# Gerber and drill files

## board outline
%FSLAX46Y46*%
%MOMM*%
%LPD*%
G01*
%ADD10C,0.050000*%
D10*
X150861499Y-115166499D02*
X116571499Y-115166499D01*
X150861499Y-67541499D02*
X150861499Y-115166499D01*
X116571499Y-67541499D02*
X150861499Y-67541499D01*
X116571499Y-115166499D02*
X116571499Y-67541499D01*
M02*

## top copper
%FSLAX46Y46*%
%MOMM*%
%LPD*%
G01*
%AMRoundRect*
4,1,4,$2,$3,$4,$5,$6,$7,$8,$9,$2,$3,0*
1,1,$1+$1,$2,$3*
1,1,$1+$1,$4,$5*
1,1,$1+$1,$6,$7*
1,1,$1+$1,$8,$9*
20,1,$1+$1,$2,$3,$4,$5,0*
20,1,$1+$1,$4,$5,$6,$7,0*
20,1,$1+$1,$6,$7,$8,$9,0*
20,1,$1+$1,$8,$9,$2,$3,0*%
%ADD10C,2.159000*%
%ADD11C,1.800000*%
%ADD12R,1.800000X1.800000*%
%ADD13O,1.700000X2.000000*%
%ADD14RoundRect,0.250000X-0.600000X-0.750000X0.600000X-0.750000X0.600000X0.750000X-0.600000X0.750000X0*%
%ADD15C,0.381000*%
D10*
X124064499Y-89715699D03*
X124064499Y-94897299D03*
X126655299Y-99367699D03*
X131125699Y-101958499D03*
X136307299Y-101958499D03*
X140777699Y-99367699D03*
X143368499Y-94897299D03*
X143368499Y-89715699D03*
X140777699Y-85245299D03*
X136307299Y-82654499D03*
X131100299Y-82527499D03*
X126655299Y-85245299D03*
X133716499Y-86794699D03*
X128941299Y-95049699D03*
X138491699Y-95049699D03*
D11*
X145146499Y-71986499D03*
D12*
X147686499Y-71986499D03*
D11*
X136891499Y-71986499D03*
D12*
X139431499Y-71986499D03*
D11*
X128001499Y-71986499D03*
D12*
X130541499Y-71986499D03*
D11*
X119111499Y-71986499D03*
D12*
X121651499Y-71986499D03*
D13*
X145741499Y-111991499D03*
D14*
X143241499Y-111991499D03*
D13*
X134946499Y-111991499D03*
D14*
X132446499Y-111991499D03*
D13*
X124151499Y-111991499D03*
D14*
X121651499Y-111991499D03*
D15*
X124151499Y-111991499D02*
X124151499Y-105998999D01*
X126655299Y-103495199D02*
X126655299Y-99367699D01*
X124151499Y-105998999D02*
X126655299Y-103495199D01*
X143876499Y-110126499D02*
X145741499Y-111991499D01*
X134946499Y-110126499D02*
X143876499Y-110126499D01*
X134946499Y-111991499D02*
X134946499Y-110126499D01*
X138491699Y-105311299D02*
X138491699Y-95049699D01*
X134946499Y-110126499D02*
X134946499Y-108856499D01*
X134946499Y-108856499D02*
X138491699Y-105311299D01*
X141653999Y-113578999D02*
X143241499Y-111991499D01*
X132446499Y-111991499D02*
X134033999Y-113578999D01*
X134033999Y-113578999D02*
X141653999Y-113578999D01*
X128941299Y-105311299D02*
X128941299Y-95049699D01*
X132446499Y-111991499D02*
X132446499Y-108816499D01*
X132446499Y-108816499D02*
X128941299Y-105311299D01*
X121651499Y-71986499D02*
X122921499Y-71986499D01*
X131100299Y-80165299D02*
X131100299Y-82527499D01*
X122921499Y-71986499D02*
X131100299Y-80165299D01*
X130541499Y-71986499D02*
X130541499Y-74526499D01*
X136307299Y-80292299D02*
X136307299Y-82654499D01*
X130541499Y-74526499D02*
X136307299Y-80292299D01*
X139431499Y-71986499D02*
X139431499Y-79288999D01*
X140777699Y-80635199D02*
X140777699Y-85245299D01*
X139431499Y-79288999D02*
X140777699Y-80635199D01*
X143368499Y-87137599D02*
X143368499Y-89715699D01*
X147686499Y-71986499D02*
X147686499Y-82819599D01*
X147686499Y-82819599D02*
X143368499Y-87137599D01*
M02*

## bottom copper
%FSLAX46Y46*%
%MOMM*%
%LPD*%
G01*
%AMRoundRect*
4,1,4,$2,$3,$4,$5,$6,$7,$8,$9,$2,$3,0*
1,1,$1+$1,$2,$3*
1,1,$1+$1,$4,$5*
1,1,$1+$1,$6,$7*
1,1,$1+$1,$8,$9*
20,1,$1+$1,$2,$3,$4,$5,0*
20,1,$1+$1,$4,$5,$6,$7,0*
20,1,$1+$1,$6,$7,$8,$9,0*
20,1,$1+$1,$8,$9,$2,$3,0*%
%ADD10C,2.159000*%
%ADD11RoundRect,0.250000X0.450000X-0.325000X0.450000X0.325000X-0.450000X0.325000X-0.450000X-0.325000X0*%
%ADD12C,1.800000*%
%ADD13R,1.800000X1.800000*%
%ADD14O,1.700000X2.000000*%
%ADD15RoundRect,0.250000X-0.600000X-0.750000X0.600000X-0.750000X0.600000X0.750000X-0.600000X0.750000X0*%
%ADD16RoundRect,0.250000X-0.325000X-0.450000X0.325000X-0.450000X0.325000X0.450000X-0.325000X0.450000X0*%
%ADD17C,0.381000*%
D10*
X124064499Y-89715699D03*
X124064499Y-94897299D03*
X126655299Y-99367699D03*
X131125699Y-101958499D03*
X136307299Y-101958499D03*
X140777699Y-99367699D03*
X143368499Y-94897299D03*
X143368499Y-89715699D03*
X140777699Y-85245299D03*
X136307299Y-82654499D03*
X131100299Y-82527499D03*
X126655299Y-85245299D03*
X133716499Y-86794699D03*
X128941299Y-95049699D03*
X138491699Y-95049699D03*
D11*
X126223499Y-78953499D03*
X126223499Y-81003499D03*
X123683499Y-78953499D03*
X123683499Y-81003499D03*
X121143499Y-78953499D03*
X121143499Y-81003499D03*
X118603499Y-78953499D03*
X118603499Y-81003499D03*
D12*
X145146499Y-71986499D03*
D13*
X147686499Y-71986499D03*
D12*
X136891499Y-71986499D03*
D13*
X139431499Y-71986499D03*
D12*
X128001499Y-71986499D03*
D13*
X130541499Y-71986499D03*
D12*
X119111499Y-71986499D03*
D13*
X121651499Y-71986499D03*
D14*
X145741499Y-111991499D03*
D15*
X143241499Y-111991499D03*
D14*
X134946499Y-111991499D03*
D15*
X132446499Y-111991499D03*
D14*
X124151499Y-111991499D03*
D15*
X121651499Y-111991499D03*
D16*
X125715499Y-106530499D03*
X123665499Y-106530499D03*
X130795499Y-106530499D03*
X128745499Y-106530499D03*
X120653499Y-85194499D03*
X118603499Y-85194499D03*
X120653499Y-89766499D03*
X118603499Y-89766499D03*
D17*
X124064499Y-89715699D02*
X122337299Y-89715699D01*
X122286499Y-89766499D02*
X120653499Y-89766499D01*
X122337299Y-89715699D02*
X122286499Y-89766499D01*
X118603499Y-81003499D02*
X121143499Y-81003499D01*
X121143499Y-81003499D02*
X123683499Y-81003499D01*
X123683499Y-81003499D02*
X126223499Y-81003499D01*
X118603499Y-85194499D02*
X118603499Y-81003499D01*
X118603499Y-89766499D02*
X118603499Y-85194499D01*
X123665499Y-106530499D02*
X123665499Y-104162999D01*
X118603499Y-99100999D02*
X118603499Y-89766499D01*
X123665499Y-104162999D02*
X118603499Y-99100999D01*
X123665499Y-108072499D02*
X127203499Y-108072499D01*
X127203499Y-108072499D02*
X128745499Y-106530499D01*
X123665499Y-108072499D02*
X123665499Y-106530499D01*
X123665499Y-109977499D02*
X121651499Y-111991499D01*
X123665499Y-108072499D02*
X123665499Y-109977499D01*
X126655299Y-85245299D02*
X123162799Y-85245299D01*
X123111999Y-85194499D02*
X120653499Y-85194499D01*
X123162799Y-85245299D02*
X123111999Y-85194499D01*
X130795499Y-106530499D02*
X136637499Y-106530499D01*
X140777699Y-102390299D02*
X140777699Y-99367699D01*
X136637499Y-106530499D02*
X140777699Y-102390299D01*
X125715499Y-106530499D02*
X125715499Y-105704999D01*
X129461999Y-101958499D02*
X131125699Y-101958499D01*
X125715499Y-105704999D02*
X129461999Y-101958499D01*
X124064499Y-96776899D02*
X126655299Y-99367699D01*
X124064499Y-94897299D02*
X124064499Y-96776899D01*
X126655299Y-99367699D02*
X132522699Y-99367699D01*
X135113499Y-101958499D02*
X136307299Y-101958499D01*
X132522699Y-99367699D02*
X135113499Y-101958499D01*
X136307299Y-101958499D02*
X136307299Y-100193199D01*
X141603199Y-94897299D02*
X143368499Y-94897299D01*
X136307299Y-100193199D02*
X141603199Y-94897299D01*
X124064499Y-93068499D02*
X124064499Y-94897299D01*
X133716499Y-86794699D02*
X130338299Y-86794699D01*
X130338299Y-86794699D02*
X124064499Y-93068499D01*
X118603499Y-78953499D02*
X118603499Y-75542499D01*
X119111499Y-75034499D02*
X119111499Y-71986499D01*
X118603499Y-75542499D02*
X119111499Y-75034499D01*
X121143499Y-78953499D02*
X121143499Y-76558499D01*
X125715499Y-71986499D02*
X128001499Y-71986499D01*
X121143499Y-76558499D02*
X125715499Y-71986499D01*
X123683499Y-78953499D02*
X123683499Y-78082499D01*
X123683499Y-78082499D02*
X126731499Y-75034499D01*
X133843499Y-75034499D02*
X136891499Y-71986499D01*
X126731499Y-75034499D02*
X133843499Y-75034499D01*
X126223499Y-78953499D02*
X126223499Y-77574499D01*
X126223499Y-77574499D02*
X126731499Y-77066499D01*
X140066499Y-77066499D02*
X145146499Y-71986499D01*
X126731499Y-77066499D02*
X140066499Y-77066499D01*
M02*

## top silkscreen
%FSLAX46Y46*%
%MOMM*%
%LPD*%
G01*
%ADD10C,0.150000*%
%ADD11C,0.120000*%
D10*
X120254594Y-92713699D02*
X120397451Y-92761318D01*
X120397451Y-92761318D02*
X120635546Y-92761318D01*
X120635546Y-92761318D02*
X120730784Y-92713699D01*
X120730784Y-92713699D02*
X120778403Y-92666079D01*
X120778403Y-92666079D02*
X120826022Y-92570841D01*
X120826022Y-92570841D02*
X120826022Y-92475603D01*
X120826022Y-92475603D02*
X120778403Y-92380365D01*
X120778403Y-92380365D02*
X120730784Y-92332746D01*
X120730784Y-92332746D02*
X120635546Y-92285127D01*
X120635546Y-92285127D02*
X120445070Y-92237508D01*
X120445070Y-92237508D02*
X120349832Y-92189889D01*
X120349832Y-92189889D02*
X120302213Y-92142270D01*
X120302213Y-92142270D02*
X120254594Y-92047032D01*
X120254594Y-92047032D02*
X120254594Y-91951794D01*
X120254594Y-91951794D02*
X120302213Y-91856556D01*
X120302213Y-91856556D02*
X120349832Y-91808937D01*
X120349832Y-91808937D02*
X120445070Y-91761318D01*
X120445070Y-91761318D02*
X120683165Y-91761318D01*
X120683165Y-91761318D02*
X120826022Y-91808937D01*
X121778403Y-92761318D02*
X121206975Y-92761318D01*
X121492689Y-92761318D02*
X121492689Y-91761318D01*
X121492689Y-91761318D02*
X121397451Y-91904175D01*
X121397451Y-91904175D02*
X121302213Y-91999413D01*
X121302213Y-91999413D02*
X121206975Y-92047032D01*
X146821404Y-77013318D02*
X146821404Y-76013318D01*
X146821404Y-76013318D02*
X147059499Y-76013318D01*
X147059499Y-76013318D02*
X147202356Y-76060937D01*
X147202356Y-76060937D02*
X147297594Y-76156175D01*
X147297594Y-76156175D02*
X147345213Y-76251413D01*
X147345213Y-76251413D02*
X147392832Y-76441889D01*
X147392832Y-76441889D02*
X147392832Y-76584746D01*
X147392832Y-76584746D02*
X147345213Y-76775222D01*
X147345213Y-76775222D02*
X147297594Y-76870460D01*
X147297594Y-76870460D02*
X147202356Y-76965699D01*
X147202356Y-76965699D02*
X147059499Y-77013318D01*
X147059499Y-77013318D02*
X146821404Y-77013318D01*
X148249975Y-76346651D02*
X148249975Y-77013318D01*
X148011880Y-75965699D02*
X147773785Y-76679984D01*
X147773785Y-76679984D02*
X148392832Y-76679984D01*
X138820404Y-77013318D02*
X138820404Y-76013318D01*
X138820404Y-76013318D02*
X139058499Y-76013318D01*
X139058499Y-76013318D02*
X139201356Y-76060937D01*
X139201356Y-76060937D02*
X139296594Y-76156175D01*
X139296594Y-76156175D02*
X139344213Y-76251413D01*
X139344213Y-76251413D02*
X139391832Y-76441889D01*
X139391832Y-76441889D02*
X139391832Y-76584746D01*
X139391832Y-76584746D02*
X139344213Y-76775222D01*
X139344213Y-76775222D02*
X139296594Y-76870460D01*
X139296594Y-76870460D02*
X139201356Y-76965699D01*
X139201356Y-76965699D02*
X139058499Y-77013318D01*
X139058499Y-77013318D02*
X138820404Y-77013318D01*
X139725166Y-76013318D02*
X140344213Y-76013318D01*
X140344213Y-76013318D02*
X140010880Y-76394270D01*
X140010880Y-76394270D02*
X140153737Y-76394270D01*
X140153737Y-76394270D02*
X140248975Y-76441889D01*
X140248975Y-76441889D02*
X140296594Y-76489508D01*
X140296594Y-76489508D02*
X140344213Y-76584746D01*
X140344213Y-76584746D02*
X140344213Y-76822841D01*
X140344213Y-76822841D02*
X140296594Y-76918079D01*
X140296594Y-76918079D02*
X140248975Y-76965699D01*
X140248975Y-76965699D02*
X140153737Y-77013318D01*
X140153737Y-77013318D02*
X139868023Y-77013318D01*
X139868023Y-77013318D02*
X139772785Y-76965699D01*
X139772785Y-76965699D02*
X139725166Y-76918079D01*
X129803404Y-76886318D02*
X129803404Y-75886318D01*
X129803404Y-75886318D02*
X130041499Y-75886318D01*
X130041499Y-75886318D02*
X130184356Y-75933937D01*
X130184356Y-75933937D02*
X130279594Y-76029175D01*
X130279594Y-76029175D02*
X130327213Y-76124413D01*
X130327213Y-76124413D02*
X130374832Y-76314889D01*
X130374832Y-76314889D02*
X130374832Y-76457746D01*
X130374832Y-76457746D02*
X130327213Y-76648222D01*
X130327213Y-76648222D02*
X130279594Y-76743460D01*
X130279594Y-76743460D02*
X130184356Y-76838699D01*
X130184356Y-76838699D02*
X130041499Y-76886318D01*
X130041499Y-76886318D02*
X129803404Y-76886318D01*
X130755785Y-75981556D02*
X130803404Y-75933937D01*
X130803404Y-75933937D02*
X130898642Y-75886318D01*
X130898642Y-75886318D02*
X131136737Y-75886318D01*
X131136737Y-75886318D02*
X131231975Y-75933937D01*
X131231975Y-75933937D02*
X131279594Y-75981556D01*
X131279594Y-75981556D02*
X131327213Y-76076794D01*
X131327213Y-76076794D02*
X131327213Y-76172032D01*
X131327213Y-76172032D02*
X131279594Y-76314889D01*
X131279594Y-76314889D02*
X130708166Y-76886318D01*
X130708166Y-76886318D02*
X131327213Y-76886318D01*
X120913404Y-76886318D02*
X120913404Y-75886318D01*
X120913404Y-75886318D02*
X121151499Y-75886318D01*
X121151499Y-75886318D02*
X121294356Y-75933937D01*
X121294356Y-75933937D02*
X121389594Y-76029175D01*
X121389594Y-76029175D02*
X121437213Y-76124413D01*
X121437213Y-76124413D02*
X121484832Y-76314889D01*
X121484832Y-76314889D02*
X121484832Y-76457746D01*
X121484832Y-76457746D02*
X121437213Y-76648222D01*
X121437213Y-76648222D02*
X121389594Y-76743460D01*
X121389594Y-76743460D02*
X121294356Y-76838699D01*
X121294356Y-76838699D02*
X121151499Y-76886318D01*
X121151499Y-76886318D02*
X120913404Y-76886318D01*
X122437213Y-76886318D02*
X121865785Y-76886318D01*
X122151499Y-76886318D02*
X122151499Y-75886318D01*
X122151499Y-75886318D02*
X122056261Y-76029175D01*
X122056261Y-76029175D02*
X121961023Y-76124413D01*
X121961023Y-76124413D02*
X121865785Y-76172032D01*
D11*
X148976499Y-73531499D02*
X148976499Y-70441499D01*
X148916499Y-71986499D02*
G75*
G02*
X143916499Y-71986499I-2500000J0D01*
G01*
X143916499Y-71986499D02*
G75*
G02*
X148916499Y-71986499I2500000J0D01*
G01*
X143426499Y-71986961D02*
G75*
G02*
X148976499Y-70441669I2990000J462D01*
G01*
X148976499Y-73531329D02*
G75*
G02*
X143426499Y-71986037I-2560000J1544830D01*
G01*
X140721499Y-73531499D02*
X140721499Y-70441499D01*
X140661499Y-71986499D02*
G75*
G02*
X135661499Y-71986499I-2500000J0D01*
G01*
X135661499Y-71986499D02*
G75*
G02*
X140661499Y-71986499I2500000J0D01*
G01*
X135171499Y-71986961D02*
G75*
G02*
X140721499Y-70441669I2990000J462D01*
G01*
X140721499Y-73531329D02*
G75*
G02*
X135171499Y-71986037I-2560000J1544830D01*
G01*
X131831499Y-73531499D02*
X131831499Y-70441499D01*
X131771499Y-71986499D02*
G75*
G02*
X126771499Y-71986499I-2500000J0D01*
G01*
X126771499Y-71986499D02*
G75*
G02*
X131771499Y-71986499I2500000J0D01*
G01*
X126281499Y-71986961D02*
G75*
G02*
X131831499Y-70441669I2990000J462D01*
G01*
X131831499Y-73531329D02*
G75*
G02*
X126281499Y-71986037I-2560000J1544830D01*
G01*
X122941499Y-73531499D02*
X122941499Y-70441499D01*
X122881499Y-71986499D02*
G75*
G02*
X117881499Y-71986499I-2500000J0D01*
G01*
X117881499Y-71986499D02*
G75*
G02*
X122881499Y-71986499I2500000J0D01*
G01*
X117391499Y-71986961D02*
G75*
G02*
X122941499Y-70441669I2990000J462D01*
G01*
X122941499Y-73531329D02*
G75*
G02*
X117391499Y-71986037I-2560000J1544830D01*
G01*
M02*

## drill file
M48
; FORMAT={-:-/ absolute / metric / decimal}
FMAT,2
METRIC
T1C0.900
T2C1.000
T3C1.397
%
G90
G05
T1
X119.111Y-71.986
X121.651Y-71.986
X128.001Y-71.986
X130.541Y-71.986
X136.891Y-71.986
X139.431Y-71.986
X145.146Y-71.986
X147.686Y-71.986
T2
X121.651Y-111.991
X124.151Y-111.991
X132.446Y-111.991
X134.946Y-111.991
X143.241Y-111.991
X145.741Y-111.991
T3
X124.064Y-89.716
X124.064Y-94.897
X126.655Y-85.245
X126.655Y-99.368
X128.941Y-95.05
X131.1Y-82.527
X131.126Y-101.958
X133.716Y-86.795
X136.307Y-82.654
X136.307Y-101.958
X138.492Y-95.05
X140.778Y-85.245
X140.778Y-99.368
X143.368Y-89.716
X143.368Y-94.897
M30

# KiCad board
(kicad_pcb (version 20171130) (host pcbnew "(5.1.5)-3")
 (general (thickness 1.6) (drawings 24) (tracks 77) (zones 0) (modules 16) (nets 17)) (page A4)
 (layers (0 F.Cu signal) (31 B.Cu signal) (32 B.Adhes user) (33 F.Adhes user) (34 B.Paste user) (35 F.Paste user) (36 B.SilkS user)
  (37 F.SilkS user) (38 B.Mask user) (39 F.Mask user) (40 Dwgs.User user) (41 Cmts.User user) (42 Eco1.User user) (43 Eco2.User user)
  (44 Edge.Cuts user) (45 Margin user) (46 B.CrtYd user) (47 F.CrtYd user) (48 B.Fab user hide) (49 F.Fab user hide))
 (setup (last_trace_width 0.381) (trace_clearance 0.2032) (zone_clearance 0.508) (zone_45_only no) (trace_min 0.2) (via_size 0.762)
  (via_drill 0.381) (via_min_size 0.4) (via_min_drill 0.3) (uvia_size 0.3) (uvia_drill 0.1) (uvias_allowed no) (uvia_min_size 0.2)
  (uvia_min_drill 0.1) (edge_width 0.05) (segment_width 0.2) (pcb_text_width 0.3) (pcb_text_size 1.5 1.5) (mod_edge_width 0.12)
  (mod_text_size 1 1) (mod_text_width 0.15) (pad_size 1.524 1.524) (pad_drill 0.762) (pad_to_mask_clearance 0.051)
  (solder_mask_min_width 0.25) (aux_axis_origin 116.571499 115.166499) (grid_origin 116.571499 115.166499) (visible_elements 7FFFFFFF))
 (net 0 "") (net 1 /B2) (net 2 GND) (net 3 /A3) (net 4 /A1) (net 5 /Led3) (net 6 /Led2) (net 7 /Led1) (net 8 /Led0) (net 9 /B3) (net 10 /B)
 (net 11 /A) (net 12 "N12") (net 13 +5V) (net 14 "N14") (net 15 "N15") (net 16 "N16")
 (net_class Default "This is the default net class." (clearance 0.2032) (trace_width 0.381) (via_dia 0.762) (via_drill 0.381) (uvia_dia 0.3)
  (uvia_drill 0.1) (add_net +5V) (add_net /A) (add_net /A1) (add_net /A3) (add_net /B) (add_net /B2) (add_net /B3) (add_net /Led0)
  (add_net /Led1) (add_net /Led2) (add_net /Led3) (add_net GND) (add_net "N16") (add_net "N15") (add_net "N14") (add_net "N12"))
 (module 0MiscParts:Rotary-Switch (layer F.Cu) (at 133.716499 92.306499)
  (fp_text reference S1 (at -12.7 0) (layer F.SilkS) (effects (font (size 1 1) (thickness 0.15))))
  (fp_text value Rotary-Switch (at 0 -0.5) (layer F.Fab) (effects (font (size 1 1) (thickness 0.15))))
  (pad 14 thru_hole circle (at -9.652 -2.5908) (size 2.159 2.159) (drill 1.397) (layers *.Cu *.Mask) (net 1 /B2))
  (pad 13 thru_hole circle (at -9.652 2.5908) (size 2.159 2.159) (drill 1.397) (layers *.Cu *.Mask) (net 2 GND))
  (pad 12 thru_hole circle (at -7.0612 7.0612) (size 2.159 2.159) (drill 1.397) (layers *.Cu *.Mask) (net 2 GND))
  (pad 10 thru_hole circle (at -2.5908 9.652) (size 2.159 2.159) (drill 1.397) (layers *.Cu *.Mask) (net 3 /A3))
  (pad 9 thru_hole circle (at 2.5908 9.652) (size 2.159 2.159) (drill 1.397) (layers *.Cu *.Mask) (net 2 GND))
  (pad 8 thru_hole circle (at 7.0612 7.0612) (size 2.159 2.159) (drill 1.397) (layers *.Cu *.Mask) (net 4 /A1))
  (pad 7 thru_hole circle (at 9.652 2.5908) (size 2.159 2.159) (drill 1.397) (layers *.Cu *.Mask) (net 2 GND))
  (pad 5 thru_hole circle (at 9.652 -2.5908) (size 2.159 2.159) (drill 1.397) (layers *.Cu *.Mask) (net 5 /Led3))
  (pad 4 thru_hole circle (at 7.0612 -7.0612) (size 2.159 2.159) (drill 1.397) (layers *.Cu *.Mask) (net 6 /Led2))
  (pad 3 thru_hole circle (at 2.5908 -9.652) (size 2.159 2.159) (drill 1.397) (layers *.Cu *.Mask) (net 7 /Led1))
  (pad 2 thru_hole circle (at -2.6162 -9.779) (size 2.159 2.159) (drill 1.397) (layers *.Cu *.Mask) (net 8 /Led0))
  (pad 15 thru_hole circle (at -7.0612 -7.0612) (size 2.159 2.159) (drill 1.397) (layers *.Cu *.Mask) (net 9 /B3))
  (pad 1 thru_hole circle (at 0 -5.5118) (size 2.159 2.159) (drill 1.397) (layers *.Cu *.Mask) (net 2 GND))
  (pad 11 thru_hole circle (at -4.7752 2.7432) (size 2.159 2.159) (drill 1.397) (layers *.Cu *.Mask) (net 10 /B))
  (pad 6 thru_hole circle (at 4.7752 2.7432) (size 2.159 2.159) (drill 1.397) (layers *.Cu *.Mask) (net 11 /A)))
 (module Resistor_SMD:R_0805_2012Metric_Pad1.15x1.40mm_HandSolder (layer B.Cu) (at 126.223499 79.978499 90)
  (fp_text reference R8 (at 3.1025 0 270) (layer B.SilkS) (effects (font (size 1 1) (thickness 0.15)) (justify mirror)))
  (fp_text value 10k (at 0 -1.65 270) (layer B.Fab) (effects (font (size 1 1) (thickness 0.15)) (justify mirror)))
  (pad 2 smd roundrect (at 1.025 0 90) (size 1.15 1.4) (layers B.Cu B.Paste B.Mask) (roundrect_rratio 0.217391) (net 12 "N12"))
  (pad 1 smd roundrect (at -1.025 0 90) (size 1.15 1.4) (layers B.Cu B.Paste B.Mask) (roundrect_rratio 0.217391) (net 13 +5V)))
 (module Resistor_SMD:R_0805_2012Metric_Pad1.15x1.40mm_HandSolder (layer B.Cu) (at 123.683499 79.978499 90)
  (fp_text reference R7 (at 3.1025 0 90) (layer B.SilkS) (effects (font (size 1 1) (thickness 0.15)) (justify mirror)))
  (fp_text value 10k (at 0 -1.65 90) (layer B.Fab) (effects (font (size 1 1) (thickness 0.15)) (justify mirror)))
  (pad 2 smd roundrect (at 1.025 0 90) (size 1.15 1.4) (layers B.Cu B.Paste B.Mask) (roundrect_rratio 0.217391) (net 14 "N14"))
  (pad 1 smd roundrect (at -1.025 0 90) (size 1.15 1.4) (layers B.Cu B.Paste B.Mask) (roundrect_rratio 0.217391) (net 13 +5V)))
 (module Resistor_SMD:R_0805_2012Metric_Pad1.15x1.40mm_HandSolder (layer B.Cu) (at 121.143499 79.978499 90)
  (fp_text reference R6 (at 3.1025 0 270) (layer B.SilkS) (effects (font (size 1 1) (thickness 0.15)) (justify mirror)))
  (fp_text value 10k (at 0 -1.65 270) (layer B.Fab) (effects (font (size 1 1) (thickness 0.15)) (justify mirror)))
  (pad 2 smd roundrect (at 1.025 0 90) (size 1.15 1.4) (layers B.Cu B.Paste B.Mask) (roundrect_rratio 0.217391) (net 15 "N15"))
  (pad 1 smd roundrect (at -1.025 0 90) (size 1.15 1.4) (layers B.Cu B.Paste B.Mask) (roundrect_rratio 0.217391) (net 13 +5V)))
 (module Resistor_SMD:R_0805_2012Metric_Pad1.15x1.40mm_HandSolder (layer B.Cu) (at 118.603499 79.978499 90)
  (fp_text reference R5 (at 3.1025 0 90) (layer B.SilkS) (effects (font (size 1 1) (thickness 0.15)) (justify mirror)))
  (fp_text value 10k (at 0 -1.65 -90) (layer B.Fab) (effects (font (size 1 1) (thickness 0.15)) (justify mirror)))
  (pad 2 smd roundrect (at 1.025 0 90) (size 1.15 1.4) (layers B.Cu B.Paste B.Mask) (roundrect_rratio 0.217391) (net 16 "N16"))
  (pad 1 smd roundrect (at -1.025 0 90) (size 1.15 1.4) (layers B.Cu B.Paste B.Mask) (roundrect_rratio 0.217391) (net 13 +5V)))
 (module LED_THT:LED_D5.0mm (layer F.Cu) (at 147.686499 71.986499 180)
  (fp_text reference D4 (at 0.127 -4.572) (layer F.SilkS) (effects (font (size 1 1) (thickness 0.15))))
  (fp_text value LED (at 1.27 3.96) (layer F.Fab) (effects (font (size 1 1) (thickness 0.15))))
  (fp_line (start -1.29 -1.545) (end -1.29 1.545) (layer F.SilkS) (width 0.12))
  (fp_circle (center 1.27 0) (end 3.77 0) (layer F.SilkS) (width 0.12))
  (fp_arc (start 1.27 0) (end -1.29 1.54483) (angle -148.9) (layer F.SilkS) (width 0.12))
  (fp_arc (start 1.27 0) (end -1.29 -1.54483) (angle 148.9) (layer F.SilkS) (width 0.12))
  (pad 2 thru_hole circle (at 2.54 0 180) (size 1.8 1.8) (drill 0.9) (layers *.Cu *.Mask) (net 12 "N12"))
  (pad 1 thru_hole rect (at 0 0 180) (size 1.8 1.8) (drill 0.9) (layers *.Cu *.Mask) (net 5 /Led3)))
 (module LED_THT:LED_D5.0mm (layer F.Cu) (at 139.431499 71.986499 180)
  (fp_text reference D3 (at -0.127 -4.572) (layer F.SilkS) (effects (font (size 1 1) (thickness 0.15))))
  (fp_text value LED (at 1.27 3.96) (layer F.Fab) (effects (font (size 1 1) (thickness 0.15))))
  (fp_line (start -1.29 -1.545) (end -1.29 1.545) (layer F.SilkS) (width 0.12))
  (fp_circle (center 1.27 0) (end 3.77 0) (layer F.SilkS) (width 0.12))
  (fp_arc (start 1.27 0) (end -1.29 1.54483) (angle -148.9) (layer F.SilkS) (width 0.12))
  (fp_arc (start 1.27 0) (end -1.29 -1.54483) (angle 148.9) (layer F.SilkS) (width 0.12))
  (pad 2 thru_hole circle (at 2.54 0 180) (size 1.8 1.8) (drill 0.9) (layers *.Cu *.Mask) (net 14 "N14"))
  (pad 1 thru_hole rect (at 0 0 180) (size 1.8 1.8) (drill 0.9) (layers *.Cu *.Mask) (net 6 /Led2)))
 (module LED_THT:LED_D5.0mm (layer F.Cu) (at 130.541499 71.986499 180)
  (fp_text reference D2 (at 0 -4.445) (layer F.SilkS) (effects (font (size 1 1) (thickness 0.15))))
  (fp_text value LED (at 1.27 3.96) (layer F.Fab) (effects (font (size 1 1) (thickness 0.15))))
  (fp_line (start -1.29 -1.545) (end -1.29 1.545) (layer F.SilkS) (width 0.12))
  (fp_circle (center 1.27 0) (end 3.77 0) (layer F.SilkS) (width 0.12))
  (fp_arc (start 1.27 0) (end -1.29 1.54483) (angle -148.9) (layer F.SilkS) (width 0.12))
  (fp_arc (start 1.27 0) (end -1.29 -1.54483) (angle 148.9) (layer F.SilkS) (width 0.12))
  (pad 2 thru_hole circle (at 2.54 0 180) (size 1.8 1.8) (drill 0.9) (layers *.Cu *.Mask) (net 15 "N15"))
  (pad 1 thru_hole rect (at 0 0 180) (size 1.8 1.8) (drill 0.9) (layers *.Cu *.Mask) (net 7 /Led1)))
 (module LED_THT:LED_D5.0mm (layer F.Cu) (at 121.651499 71.986499 180)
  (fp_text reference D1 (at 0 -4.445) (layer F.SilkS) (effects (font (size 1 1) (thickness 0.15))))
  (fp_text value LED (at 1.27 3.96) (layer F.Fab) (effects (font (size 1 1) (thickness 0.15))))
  (fp_line (start -1.29 -1.545) (end -1.29 1.545) (layer F.SilkS) (width 0.12))
  (fp_circle (center 1.27 0) (end 3.77 0) (layer F.SilkS) (width 0.12))
  (fp_arc (start 1.27 0) (end -1.29 1.54483) (angle -148.9) (layer F.SilkS) (width 0.12))
  (fp_arc (start 1.27 0) (end -1.29 -1.54483) (angle 148.9) (layer F.SilkS) (width 0.12))
  (pad 2 thru_hole circle (at 2.54 0 180) (size 1.8 1.8) (drill 0.9) (layers *.Cu *.Mask) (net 16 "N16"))
  (pad 1 thru_hole rect (at 0 0 180) (size 1.8 1.8) (drill 0.9) (layers *.Cu *.Mask) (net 8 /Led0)))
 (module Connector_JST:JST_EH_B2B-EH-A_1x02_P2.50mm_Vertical (layer B.Cu) (at 143.241499 111.991499)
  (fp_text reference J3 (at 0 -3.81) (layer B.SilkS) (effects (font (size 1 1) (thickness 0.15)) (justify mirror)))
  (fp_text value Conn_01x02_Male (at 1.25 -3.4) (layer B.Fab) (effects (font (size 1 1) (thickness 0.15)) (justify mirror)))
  (pad 2 thru_hole oval (at 2.5 0) (size 1.7 2) (drill 1) (layers *.Cu *.Mask) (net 11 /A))
  (pad 1 thru_hole roundrect (at 0 0) (size 1.7 2) (drill 1) (layers *.Cu *.Mask) (roundrect_rratio 0.147059) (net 10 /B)))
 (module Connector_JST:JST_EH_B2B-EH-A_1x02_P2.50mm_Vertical (layer B.Cu) (at 132.446499 111.991499)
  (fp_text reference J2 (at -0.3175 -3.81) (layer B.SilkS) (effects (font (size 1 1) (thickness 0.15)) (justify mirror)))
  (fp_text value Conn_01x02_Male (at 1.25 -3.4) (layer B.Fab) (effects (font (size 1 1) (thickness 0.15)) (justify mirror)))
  (pad 2 thru_hole oval (at 2.5 0) (size 1.7 2) (drill 1) (layers *.Cu *.Mask) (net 11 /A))
  (pad 1 thru_hole roundrect (at 0 0) (size 1.7 2) (drill 1) (layers *.Cu *.Mask) (roundrect_rratio 0.147059) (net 10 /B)))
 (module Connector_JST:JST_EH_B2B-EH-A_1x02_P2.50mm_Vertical (layer B.Cu) (at 121.651499 111.991499)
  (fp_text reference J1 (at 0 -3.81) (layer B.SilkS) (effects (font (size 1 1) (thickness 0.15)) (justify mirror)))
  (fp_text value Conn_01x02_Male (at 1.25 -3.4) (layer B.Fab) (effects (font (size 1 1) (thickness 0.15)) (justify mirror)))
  (pad 2 thru_hole oval (at 2.5 0) (size 1.7 2) (drill 1) (layers *.Cu *.Mask) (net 2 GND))
  (pad 1 thru_hole roundrect (at 0 0) (size 1.7 2) (drill 1) (layers *.Cu *.Mask) (roundrect_rratio 0.147059) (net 13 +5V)))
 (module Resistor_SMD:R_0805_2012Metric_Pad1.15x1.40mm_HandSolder (layer B.Cu) (at 124.690499 106.530499)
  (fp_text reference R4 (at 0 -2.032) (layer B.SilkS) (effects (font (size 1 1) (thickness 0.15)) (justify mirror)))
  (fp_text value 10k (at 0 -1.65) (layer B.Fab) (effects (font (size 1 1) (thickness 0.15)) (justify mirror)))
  (pad 2 smd roundrect (at 1.025 0) (size 1.15 1.4) (layers B.Cu B.Paste B.Mask) (roundrect_rratio 0.217391) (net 3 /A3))
  (pad 1 smd roundrect (at -1.025 0) (size 1.15 1.4) (layers B.Cu B.Paste B.Mask) (roundrect_rratio 0.217391) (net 13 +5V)))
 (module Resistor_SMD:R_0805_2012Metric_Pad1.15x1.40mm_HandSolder (layer B.Cu) (at 129.770499 106.530499)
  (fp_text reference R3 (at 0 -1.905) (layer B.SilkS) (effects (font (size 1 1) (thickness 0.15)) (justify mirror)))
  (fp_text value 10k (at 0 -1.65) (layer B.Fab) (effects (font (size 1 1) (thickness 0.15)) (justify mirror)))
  (pad 2 smd roundrect (at 1.025 0) (size 1.15 1.4) (layers B.Cu B.Paste B.Mask) (roundrect_rratio 0.217391) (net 4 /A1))
  (pad 1 smd roundrect (at -1.025 0) (size 1.15 1.4) (layers B.Cu B.Paste B.Mask) (roundrect_rratio 0.217391) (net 13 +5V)))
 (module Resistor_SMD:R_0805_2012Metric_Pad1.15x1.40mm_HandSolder (layer B.Cu) (at 119.628499 85.194499)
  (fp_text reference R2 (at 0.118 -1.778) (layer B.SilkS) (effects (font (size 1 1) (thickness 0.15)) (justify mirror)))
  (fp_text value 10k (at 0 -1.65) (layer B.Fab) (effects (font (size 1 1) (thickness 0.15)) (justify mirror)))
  (pad 2 smd roundrect (at 1.025 0) (size 1.15 1.4) (layers B.Cu B.Paste B.Mask) (roundrect_rratio 0.217391) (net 9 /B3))
  (pad 1 smd roundrect (at -1.025 0) (size 1.15 1.4) (layers B.Cu B.Paste B.Mask) (roundrect_rratio 0.217391) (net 13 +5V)))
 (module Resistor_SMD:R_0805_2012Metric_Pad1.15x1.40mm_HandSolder (layer B.Cu) (at 119.628499 89.766499)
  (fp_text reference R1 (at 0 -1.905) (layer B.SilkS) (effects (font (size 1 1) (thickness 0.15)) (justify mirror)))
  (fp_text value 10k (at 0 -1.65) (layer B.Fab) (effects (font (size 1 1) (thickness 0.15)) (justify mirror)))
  (pad 2 smd roundrect (at 1.025 0) (size 1.15 1.4) (layers B.Cu B.Paste B.Mask) (roundrect_rratio 0.217391) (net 1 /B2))
  (pad 1 smd roundrect (at -1.025 0) (size 1.15 1.4) (layers B.Cu B.Paste B.Mask) (roundrect_rratio 0.217391) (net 13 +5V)))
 (gr_line (start 150.861499 115.166499) (end 116.571499 115.166499) (layer Edge.Cuts) (width 0.05))
 (gr_line (start 150.861499 67.541499) (end 150.861499 115.166499) (layer Edge.Cuts) (width 0.05))
 (gr_line (start 116.571499 67.541499) (end 150.861499 67.541499) (layer Edge.Cuts) (width 0.05))
 (gr_line (start 116.571499 115.166499) (end 116.571499 67.541499) (layer Edge.Cuts) (width 0.05))
 (segment (start 124.064499 89.715699) (end 122.337299 89.715699) (width 0.381) (layer B.Cu) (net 1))
 (segment (start 122.286499 89.766499) (end 120.653499 89.766499) (width 0.381) (layer B.Cu) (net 1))
 (segment (start 122.337299 89.715699) (end 122.286499 89.766499) (width 0.381) (layer B.Cu) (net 1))
 (segment (start 118.603499 81.003499) (end 121.143499 81.003499) (width 0.381) (layer B.Cu) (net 13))
 (segment (start 121.143499 81.003499) (end 123.683499 81.003499) (width 0.381) (layer B.Cu) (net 13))
 (segment (start 123.683499 81.003499) (end 126.223499 81.003499) (width 0.381) (layer B.Cu) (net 13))
 (segment (start 118.603499 85.194499) (end 118.603499 81.003499) (width 0.381) (layer B.Cu) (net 13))
 (segment (start 118.603499 89.766499) (end 118.603499 85.194499) (width 0.381) (layer B.Cu) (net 13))
 (segment (start 123.665499 106.530499) (end 123.665499 104.162999) (width 0.381) (layer B.Cu) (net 13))
 (segment (start 118.603499 99.100999) (end 118.603499 89.766499) (width 0.381) (layer B.Cu) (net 13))
 (segment (start 123.665499 104.162999) (end 118.603499 99.100999) (width 0.381) (layer B.Cu) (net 13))
 (segment (start 123.665499 108.072499) (end 127.203499 108.072499) (width 0.381) (layer B.Cu) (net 13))
 (segment (start 127.203499 108.072499) (end 128.745499 106.530499) (width 0.381) (layer B.Cu) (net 13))
 (segment (start 123.665499 108.072499) (end 123.665499 106.530499) (width 0.381) (layer B.Cu) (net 13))
 (segment (start 123.665499 109.977499) (end 121.651499 111.991499) (width 0.381) (layer B.Cu) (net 13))
 (segment (start 123.665499 108.072499) (end 123.665499 109.977499) (width 0.381) (layer B.Cu) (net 13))
 (segment (start 126.655299 85.245299) (end 123.162799 85.245299) (width 0.381) (layer B.Cu) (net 9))
 (segment (start 123.111999 85.194499) (end 120.653499 85.194499) (width 0.381) (layer B.Cu) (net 9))
 (segment (start 123.162799 85.245299) (end 123.111999 85.194499) (width 0.381) (layer B.Cu) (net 9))
 (segment (start 130.795499 106.530499) (end 136.637499 106.530499) (width 0.381) (layer B.Cu) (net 4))
 (segment (start 140.777699 102.390299) (end 140.777699 99.367699) (width 0.381) (layer B.Cu) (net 4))
 (segment (start 136.637499 106.530499) (end 140.777699 102.390299) (width 0.381) (layer B.Cu) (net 4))
 (segment (start 125.715499 106.530499) (end 125.715499 105.704999) (width 0.381) (layer B.Cu) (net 3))
 (segment (start 129.461999 101.958499) (end 131.125699 101.958499) (width 0.381) (layer B.Cu) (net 3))
 (segment (start 125.715499 105.704999) (end 129.461999 101.958499) (width 0.381) (layer B.Cu) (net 3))
 (segment (start 124.064499 96.776899) (end 126.655299 99.367699) (width 0.381) (layer B.Cu) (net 2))
 (segment (start 124.064499 94.897299) (end 124.064499 96.776899) (width 0.381) (layer B.Cu) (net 2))
 (segment (start 126.655299 99.367699) (end 132.522699 99.367699) (width 0.381) (layer B.Cu) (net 2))
 (segment (start 135.113499 101.958499) (end 136.307299 101.958499) (width 0.381) (layer B.Cu) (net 2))
 (segment (start 132.522699 99.367699) (end 135.113499 101.958499) (width 0.381) (layer B.Cu) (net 2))
 (segment (start 136.307299 101.958499) (end 136.307299 100.193199) (width 0.381) (layer B.Cu) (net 2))
 (segment (start 141.603199 94.897299) (end 143.368499 94.897299) (width 0.381) (layer B.Cu) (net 2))
 (segment (start 136.307299 100.193199) (end 141.603199 94.897299) (width 0.381) (layer B.Cu) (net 2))
 (segment (start 124.151499 111.991499) (end 124.151499 105.998999) (width 0.381) (layer F.Cu) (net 2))
 (segment (start 126.655299 103.495199) (end 126.655299 99.367699) (width 0.381) (layer F.Cu) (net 2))
 (segment (start 124.151499 105.998999) (end 126.655299 103.495199) (width 0.381) (layer F.Cu) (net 2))
 (segment (start 124.064499 93.068499) (end 124.064499 94.897299) (width 0.381) (layer B.Cu) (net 2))
 (segment (start 133.716499 86.794699) (end 130.338299 86.794699) (width 0.381) (layer B.Cu) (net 2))
 (segment (start 130.338299 86.794699) (end 124.064499 93.068499) (width 0.381) (layer B.Cu) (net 2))
 (segment (start 143.876499 110.126499) (end 145.741499 111.991499) (width 0.381) (layer F.Cu) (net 11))
 (segment (start 134.946499 110.126499) (end 143.876499 110.126499) (width 0.381) (layer F.Cu) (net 11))
 (segment (start 134.946499 111.991499) (end 134.946499 110.126499) (width 0.381) (layer F.Cu) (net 11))
 (segment (start 138.491699 105.311299) (end 138.491699 95.049699) (width 0.381) (layer F.Cu) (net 11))
 (segment (start 134.946499 110.126499) (end 134.946499 108.856499) (width 0.381) (layer F.Cu) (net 11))
 (segment (start 134.946499 108.856499) (end 138.491699 105.311299) (width 0.381) (layer F.Cu) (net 11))
 (segment (start 141.653999 113.578999) (end 143.241499 111.991499) (width 0.381) (layer F.Cu) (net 10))
 (segment (start 132.446499 111.991499) (end 134.033999 113.578999) (width 0.381) (layer F.Cu) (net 10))
 (segment (start 134.033999 113.578999) (end 141.653999 113.578999) (width 0.381) (layer F.Cu) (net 10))
 (segment (start 128.941299 105.311299) (end 128.941299 95.049699) (width 0.381) (layer F.Cu) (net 10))
 (segment (start 132.446499 111.991499) (end 132.446499 108.816499) (width 0.381) (layer F.Cu) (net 10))
 (segment (start 132.446499 108.816499) (end 128.941299 105.311299) (width 0.381) (layer F.Cu) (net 10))
 (segment (start 118.603499 78.953499) (end 118.603499 75.542499) (width 0.381) (layer B.Cu) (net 16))
 (segment (start 119.111499 75.034499) (end 119.111499 71.986499) (width 0.381) (layer B.Cu) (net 16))
 (segment (start 118.603499 75.542499) (end 119.111499 75.034499) (width 0.381) (layer B.Cu) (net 16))
 (segment (start 121.651499 71.986499) (end 122.921499 71.986499) (width 0.381) (layer F.Cu) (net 8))
 (segment (start 131.100299 80.165299) (end 131.100299 82.527499) (width 0.381) (layer F.Cu) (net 8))
 (segment (start 122.921499 71.986499) (end 131.100299 80.165299) (width 0.381) (layer F.Cu) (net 8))
 (segment (start 121.143499 78.953499) (end 121.143499 76.558499) (width 0.381) (layer B.Cu) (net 15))
 (segment (start 125.715499 71.986499) (end 128.001499 71.986499) (width 0.381) (layer B.Cu) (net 15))
 (segment (start 121.143499 76.558499) (end 125.715499 71.986499) (width 0.381) (layer B.Cu) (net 15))
 (segment (start 130.541499 71.986499) (end 130.541499 74.526499) (width 0.381) (layer F.Cu) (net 7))
 (segment (start 136.307299 80.292299) (end 136.307299 82.654499) (width 0.381) (layer F.Cu) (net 7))
 (segment (start 130.541499 74.526499) (end 136.307299 80.292299) (width 0.381) (layer F.Cu) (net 7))
 (segment (start 123.683499 78.953499) (end 123.683499 78.082499) (width 0.381) (layer B.Cu) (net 14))
 (segment (start 123.683499 78.082499) (end 126.731499 75.034499) (width 0.381) (layer B.Cu) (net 14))
 (segment (start 133.843499 75.034499) (end 136.891499 71.986499) (width 0.381) (layer B.Cu) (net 14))
 (segment (start 126.731499 75.034499) (end 133.843499 75.034499) (width 0.381) (layer B.Cu) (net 14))
 (segment (start 139.431499 71.986499) (end 139.431499 79.288999) (width 0.381) (layer F.Cu) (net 6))
 (segment (start 140.777699 80.635199) (end 140.777699 85.245299) (width 0.381) (layer F.Cu) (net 6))
 (segment (start 139.431499 79.288999) (end 140.777699 80.635199) (width 0.381) (layer F.Cu) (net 6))
 (segment (start 126.223499 78.953499) (end 126.223499 77.574499) (width 0.381) (layer B.Cu) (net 12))
 (segment (start 126.223499 77.574499) (end 126.731499 77.066499) (width 0.381) (layer B.Cu) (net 12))
 (segment (start 140.066499 77.066499) (end 145.146499 71.986499) (width 0.381) (layer B.Cu) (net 12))
 (segment (start 126.731499 77.066499) (end 140.066499 77.066499) (width 0.381) (layer B.Cu) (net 12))
 (segment (start 143.368499 87.137599) (end 143.368499 89.715699) (width 0.381) (layer F.Cu) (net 5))
 (segment (start 147.686499 71.986499) (end 147.686499 82.819599) (width 0.381) (layer F.Cu) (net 5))
 (segment (start 147.686499 82.819599) (end 143.368499 87.137599) (width 0.381) (layer F.Cu) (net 5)))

